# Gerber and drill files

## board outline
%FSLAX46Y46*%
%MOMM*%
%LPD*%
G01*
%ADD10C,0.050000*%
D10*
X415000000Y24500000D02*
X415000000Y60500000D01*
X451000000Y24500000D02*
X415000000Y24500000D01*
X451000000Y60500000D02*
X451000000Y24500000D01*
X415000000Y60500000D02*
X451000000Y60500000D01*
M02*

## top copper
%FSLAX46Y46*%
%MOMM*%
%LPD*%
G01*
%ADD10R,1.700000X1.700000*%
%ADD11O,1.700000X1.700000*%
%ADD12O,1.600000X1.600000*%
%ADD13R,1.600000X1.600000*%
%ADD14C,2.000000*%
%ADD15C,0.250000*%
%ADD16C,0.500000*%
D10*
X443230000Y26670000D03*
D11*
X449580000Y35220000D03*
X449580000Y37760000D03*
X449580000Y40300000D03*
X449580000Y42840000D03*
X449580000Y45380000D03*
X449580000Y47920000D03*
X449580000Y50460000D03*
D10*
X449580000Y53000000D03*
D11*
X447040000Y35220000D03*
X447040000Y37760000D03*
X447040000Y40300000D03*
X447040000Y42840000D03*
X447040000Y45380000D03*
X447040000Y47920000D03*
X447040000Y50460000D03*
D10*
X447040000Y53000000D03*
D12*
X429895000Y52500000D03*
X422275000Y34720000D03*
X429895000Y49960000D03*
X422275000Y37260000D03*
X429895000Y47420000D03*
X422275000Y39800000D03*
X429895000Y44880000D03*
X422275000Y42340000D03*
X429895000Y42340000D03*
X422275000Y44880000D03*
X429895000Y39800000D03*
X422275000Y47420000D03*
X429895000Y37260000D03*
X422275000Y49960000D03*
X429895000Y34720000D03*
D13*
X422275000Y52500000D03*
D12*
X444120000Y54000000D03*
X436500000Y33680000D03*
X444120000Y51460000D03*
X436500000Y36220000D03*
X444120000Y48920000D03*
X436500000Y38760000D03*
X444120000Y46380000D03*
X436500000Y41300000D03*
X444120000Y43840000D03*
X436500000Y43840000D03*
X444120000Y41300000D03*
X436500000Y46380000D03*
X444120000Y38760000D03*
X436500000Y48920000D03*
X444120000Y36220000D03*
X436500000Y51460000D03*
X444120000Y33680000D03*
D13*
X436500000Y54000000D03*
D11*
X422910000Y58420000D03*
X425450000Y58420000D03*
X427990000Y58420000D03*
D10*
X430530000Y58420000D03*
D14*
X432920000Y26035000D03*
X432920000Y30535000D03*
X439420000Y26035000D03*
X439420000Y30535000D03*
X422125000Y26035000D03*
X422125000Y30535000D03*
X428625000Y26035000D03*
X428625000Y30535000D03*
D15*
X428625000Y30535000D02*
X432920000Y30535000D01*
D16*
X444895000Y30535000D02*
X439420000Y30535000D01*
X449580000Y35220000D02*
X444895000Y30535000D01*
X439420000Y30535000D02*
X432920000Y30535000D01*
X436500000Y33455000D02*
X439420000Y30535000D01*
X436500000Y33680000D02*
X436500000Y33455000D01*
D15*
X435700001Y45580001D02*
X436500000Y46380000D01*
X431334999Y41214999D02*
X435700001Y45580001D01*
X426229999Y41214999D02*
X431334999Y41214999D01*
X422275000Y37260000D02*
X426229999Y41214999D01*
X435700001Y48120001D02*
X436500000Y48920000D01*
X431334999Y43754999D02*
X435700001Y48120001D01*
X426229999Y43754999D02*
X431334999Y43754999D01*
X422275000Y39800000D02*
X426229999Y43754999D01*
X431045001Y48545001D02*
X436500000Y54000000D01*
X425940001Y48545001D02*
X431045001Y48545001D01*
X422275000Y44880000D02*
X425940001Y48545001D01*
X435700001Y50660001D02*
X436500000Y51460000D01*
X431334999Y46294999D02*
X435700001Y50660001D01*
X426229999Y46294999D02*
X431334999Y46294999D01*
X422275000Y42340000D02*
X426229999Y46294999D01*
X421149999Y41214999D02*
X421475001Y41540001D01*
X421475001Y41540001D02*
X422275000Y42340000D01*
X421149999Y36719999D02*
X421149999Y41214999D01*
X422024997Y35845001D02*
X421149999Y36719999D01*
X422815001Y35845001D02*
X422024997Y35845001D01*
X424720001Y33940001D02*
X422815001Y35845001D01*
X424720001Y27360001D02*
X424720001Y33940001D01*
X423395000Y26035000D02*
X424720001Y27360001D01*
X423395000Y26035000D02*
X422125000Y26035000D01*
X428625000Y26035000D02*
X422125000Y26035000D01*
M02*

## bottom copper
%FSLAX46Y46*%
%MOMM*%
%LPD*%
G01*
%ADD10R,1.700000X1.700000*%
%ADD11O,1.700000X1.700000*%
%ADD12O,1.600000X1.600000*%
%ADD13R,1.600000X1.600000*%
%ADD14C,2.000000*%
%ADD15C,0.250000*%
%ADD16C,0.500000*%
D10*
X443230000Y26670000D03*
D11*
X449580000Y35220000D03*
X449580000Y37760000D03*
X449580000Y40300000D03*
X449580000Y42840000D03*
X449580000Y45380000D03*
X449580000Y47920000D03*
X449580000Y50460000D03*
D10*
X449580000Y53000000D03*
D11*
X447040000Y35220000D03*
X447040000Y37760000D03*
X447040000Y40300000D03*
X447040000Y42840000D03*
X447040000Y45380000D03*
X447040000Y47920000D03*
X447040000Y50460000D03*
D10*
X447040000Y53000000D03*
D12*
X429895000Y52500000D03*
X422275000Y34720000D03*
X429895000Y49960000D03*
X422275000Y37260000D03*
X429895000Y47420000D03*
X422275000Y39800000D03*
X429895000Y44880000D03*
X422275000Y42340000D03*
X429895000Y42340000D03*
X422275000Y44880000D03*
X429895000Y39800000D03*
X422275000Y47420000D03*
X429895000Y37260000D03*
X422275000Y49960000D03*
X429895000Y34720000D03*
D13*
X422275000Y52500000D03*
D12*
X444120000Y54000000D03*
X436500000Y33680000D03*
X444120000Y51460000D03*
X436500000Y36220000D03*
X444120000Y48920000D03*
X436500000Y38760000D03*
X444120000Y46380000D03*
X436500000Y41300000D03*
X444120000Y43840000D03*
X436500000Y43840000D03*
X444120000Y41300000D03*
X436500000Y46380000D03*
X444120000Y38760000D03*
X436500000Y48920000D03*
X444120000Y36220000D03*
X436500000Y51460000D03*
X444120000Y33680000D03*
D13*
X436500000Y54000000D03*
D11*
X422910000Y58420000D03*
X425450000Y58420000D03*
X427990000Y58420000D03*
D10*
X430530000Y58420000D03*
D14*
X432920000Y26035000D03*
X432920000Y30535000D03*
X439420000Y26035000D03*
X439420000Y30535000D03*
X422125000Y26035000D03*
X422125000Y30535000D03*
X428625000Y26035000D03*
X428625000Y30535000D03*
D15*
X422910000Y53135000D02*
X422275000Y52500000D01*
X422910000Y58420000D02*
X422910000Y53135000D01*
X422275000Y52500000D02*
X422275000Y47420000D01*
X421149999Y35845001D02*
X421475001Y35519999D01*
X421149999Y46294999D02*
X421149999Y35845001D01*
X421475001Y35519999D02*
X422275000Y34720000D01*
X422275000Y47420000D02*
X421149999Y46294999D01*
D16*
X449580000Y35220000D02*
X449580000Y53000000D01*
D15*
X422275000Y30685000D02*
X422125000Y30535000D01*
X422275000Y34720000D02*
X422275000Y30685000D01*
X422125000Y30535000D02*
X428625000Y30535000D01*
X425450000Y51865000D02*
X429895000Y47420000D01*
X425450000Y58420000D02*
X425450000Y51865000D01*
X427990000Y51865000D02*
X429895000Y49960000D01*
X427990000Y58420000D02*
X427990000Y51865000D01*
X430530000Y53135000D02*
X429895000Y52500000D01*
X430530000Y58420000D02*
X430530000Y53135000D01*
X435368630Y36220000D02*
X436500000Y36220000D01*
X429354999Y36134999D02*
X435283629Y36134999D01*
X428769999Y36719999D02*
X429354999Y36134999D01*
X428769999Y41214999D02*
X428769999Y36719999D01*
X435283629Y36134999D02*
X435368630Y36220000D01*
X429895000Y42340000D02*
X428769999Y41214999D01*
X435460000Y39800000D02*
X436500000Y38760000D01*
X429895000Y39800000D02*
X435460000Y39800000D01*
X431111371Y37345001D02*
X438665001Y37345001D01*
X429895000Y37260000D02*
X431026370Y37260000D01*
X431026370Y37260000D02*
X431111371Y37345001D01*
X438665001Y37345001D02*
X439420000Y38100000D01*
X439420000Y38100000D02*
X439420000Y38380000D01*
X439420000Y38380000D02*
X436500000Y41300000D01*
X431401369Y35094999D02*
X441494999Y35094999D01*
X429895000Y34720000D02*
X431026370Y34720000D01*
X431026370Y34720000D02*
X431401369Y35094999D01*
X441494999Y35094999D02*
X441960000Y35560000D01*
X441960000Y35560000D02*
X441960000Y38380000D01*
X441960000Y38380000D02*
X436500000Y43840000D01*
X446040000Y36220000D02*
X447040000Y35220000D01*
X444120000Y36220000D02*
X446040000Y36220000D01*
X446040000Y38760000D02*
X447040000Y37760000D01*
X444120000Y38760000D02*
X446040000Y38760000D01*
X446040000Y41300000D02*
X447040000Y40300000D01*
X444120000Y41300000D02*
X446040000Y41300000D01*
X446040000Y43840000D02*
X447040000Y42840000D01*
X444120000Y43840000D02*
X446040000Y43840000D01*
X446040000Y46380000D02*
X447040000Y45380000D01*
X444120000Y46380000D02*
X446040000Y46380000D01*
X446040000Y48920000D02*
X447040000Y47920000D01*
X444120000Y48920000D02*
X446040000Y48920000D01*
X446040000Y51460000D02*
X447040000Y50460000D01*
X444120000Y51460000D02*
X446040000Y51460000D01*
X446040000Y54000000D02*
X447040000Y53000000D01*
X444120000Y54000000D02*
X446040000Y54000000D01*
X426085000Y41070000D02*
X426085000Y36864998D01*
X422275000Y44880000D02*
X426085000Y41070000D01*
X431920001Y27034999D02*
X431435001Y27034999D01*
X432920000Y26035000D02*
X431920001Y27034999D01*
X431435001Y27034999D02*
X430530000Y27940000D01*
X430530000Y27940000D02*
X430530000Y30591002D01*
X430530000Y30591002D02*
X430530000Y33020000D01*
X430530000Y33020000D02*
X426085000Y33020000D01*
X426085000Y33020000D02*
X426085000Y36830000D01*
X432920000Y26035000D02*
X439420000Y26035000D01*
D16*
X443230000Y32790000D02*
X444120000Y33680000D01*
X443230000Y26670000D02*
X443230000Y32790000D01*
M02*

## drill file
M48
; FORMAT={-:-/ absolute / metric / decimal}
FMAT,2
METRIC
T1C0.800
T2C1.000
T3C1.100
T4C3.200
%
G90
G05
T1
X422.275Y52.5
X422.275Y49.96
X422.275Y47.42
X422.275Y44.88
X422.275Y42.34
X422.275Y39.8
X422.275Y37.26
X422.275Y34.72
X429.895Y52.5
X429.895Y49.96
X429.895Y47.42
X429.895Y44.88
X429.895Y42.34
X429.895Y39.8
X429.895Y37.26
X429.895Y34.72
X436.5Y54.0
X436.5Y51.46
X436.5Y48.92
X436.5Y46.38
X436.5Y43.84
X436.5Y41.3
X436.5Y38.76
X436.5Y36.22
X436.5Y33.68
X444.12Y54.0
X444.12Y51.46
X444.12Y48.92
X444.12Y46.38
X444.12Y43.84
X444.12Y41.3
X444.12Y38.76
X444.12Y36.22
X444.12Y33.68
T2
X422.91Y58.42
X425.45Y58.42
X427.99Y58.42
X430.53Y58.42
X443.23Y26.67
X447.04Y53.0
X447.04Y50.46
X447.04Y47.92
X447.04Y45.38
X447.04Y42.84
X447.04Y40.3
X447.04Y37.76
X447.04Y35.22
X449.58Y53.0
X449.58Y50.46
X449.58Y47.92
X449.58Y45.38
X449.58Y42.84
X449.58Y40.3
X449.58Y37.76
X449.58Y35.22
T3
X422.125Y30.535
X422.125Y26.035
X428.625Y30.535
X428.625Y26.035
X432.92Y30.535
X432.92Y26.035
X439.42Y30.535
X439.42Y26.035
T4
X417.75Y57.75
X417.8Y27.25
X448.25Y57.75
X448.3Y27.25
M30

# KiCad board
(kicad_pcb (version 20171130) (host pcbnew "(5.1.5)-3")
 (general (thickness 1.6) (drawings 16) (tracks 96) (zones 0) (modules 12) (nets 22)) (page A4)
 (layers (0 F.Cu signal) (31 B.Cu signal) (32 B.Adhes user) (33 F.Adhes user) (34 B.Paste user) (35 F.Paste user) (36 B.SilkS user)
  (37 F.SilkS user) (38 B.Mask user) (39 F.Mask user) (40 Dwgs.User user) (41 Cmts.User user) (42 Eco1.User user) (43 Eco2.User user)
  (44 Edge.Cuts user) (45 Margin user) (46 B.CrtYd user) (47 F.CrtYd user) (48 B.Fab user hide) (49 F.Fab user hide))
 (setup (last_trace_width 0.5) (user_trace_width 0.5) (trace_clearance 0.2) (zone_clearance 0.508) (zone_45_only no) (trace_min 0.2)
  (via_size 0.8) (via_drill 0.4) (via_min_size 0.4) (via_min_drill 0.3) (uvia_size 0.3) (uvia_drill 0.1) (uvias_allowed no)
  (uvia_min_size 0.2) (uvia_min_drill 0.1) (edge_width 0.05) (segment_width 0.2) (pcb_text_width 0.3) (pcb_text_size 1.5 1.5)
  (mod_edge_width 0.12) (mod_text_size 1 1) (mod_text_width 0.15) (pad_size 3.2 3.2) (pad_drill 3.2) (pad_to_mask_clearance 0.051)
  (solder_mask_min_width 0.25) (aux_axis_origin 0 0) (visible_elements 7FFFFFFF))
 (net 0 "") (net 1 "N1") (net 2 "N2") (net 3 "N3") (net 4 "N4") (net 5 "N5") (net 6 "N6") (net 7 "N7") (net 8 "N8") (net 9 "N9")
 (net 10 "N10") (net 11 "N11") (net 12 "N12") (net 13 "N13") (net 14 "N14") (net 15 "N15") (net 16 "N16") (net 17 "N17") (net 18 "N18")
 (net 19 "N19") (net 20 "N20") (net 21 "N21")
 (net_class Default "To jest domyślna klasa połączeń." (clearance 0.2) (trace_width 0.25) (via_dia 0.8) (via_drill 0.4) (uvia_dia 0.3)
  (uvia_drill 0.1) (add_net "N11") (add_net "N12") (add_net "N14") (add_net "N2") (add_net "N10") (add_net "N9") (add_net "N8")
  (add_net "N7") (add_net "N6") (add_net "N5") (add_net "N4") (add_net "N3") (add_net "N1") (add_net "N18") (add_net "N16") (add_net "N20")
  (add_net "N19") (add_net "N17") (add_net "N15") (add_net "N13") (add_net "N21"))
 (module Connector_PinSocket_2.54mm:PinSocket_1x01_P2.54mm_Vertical (layer F.Cu) (at 443.23 -26.67)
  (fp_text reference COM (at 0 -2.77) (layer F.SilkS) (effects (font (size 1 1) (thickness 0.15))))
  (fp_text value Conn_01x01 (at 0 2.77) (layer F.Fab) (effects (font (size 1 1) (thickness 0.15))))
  (pad 1 thru_hole rect (at 0 0) (size 1.7 1.7) (drill 1) (layers *.Cu *.Mask) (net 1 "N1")))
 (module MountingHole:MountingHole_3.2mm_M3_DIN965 (layer F.Cu) (at 448.3 -27.25)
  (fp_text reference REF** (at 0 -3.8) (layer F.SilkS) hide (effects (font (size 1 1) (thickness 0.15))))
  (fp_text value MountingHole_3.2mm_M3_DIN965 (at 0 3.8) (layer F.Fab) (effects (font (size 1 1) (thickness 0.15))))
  (pad "" np_thru_hole circle (at 0 0) (size 3.2 3.2) (drill 3.2) (layers *.Cu)))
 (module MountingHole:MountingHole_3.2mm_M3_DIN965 (layer F.Cu) (at 417.8 -27.25)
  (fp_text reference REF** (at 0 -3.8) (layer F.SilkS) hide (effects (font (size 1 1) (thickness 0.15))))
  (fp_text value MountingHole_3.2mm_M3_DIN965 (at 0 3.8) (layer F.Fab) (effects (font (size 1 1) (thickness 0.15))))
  (pad "" np_thru_hole circle (at 0 0) (size 3.2 3.2) (drill 3.2) (layers *.Cu)))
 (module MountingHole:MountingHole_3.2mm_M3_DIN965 (layer F.Cu) (at 448.25 -57.75)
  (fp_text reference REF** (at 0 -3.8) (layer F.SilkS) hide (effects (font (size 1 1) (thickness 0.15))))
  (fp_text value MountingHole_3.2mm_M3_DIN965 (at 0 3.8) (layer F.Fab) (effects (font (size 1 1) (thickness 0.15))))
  (pad "" np_thru_hole circle (at 0 0) (size 3.2 3.2) (drill 3.2) (layers *.Cu)))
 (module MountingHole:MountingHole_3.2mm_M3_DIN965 (layer F.Cu) (at 417.75 -57.75)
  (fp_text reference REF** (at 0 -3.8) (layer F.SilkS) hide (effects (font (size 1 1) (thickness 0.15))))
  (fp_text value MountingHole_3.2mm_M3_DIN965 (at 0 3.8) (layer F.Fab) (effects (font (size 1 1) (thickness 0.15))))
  (pad "" np_thru_hole circle (at 0 0) (size 3.2 3.2) (drill 3.2) (layers *.Cu)))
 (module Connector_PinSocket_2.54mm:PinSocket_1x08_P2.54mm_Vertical (layer F.Cu) (at 449.58 -53)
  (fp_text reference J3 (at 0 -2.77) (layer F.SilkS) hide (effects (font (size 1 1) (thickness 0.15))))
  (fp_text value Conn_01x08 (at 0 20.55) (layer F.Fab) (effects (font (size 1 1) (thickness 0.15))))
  (pad 8 thru_hole oval (at 0 17.78) (size 1.7 1.7) (drill 1) (layers *.Cu *.Mask) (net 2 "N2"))
  (pad 7 thru_hole oval (at 0 15.24) (size 1.7 1.7) (drill 1) (layers *.Cu *.Mask) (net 2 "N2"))
  (pad 6 thru_hole oval (at 0 12.7) (size 1.7 1.7) (drill 1) (layers *.Cu *.Mask) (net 2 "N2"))
  (pad 5 thru_hole oval (at 0 10.16) (size 1.7 1.7) (drill 1) (layers *.Cu *.Mask) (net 2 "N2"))
  (pad 4 thru_hole oval (at 0 7.62) (size 1.7 1.7) (drill 1) (layers *.Cu *.Mask) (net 2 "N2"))
  (pad 3 thru_hole oval (at 0 5.08) (size 1.7 1.7) (drill 1) (layers *.Cu *.Mask) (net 2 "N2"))
  (pad 2 thru_hole oval (at 0 2.54) (size 1.7 1.7) (drill 1) (layers *.Cu *.Mask) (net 2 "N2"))
  (pad 1 thru_hole rect (at 0 0) (size 1.7 1.7) (drill 1) (layers *.Cu *.Mask) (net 2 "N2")))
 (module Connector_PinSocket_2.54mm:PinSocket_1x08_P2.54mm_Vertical (layer F.Cu) (at 447.04 -53)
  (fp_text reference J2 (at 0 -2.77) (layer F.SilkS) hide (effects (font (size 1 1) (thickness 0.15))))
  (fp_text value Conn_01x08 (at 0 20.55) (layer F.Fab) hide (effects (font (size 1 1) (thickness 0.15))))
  (pad 8 thru_hole oval (at 0 17.78) (size 1.7 1.7) (drill 1) (layers *.Cu *.Mask) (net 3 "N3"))
  (pad 7 thru_hole oval (at 0 15.24) (size 1.7 1.7) (drill 1) (layers *.Cu *.Mask) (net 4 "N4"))
  (pad 6 thru_hole oval (at 0 12.7) (size 1.7 1.7) (drill 1) (layers *.Cu *.Mask) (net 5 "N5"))
  (pad 5 thru_hole oval (at 0 10.16) (size 1.7 1.7) (drill 1) (layers *.Cu *.Mask) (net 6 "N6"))
  (pad 4 thru_hole oval (at 0 7.62) (size 1.7 1.7) (drill 1) (layers *.Cu *.Mask) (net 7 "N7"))
  (pad 3 thru_hole oval (at 0 5.08) (size 1.7 1.7) (drill 1) (layers *.Cu *.Mask) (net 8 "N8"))
  (pad 2 thru_hole oval (at 0 2.54) (size 1.7 1.7) (drill 1) (layers *.Cu *.Mask) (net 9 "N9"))
  (pad 1 thru_hole rect (at 0 0) (size 1.7 1.7) (drill 1) (layers *.Cu *.Mask) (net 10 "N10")))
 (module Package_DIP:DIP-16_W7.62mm (layer F.Cu) (at 422.275 -52.5)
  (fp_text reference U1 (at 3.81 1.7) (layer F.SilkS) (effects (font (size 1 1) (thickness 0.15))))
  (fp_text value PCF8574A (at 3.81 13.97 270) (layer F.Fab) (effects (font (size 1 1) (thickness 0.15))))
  (pad 16 thru_hole oval (at 7.62 0) (size 1.6 1.6) (drill 0.8) (layers *.Cu *.Mask) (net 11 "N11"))
  (pad 8 thru_hole oval (at 0 17.78) (size 1.6 1.6) (drill 0.8) (layers *.Cu *.Mask) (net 2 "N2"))
  (pad 15 thru_hole oval (at 7.62 2.54) (size 1.6 1.6) (drill 0.8) (layers *.Cu *.Mask) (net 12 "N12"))
  (pad 7 thru_hole oval (at 0 15.24) (size 1.6 1.6) (drill 0.8) (layers *.Cu *.Mask) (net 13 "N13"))
  (pad 14 thru_hole oval (at 7.62 5.08) (size 1.6 1.6) (drill 0.8) (layers *.Cu *.Mask) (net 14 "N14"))
  (pad 6 thru_hole oval (at 0 12.7) (size 1.6 1.6) (drill 0.8) (layers *.Cu *.Mask) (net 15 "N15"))
  (pad 13 thru_hole oval (at 7.62 7.62) (size 1.6 1.6) (drill 0.8) (layers *.Cu *.Mask))
  (pad 5 thru_hole oval (at 0 10.16) (size 1.6 1.6) (drill 0.8) (layers *.Cu *.Mask) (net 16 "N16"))
  (pad 12 thru_hole oval (at 7.62 10.16) (size 1.6 1.6) (drill 0.8) (layers *.Cu *.Mask) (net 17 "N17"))
  (pad 4 thru_hole oval (at 0 7.62) (size 1.6 1.6) (drill 0.8) (layers *.Cu *.Mask) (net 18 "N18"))
  (pad 11 thru_hole oval (at 7.62 12.7) (size 1.6 1.6) (drill 0.8) (layers *.Cu *.Mask) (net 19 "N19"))
  (pad 3 thru_hole oval (at 0 5.08) (size 1.6 1.6) (drill 0.8) (layers *.Cu *.Mask) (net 2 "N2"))
  (pad 10 thru_hole oval (at 7.62 15.24) (size 1.6 1.6) (drill 0.8) (layers *.Cu *.Mask) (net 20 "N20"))
  (pad 2 thru_hole oval (at 0 2.54) (size 1.6 1.6) (drill 0.8) (layers *.Cu *.Mask) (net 2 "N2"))
  (pad 9 thru_hole oval (at 7.62 17.78) (size 1.6 1.6) (drill 0.8) (layers *.Cu *.Mask) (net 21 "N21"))
  (pad 1 thru_hole rect (at 0 0) (size 1.6 1.6) (drill 0.8) (layers *.Cu *.Mask) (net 2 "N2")))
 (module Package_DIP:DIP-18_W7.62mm (layer F.Cu) (at 436.5 -54)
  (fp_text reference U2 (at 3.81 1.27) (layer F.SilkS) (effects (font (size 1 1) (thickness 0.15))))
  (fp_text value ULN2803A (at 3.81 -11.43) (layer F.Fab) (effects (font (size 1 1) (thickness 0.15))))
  (pad 18 thru_hole oval (at 7.62 0) (size 1.6 1.6) (drill 0.8) (layers *.Cu *.Mask) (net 10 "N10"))
  (pad 9 thru_hole oval (at 0 20.32) (size 1.6 1.6) (drill 0.8) (layers *.Cu *.Mask) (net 2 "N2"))
  (pad 17 thru_hole oval (at 7.62 2.54) (size 1.6 1.6) (drill 0.8) (layers *.Cu *.Mask) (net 9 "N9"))
  (pad 8 thru_hole oval (at 0 17.78) (size 1.6 1.6) (drill 0.8) (layers *.Cu *.Mask) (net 17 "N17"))
  (pad 16 thru_hole oval (at 7.62 5.08) (size 1.6 1.6) (drill 0.8) (layers *.Cu *.Mask) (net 8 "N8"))
  (pad 7 thru_hole oval (at 0 15.24) (size 1.6 1.6) (drill 0.8) (layers *.Cu *.Mask) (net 19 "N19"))
  (pad 15 thru_hole oval (at 7.62 7.62) (size 1.6 1.6) (drill 0.8) (layers *.Cu *.Mask) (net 7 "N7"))
  (pad 6 thru_hole oval (at 0 12.7) (size 1.6 1.6) (drill 0.8) (layers *.Cu *.Mask) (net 20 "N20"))
  (pad 14 thru_hole oval (at 7.62 10.16) (size 1.6 1.6) (drill 0.8) (layers *.Cu *.Mask) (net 6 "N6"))
  (pad 5 thru_hole oval (at 0 10.16) (size 1.6 1.6) (drill 0.8) (layers *.Cu *.Mask) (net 21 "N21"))
  (pad 13 thru_hole oval (at 7.62 12.7) (size 1.6 1.6) (drill 0.8) (layers *.Cu *.Mask) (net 5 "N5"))
  (pad 4 thru_hole oval (at 0 7.62) (size 1.6 1.6) (drill 0.8) (layers *.Cu *.Mask) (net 13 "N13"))
  (pad 12 thru_hole oval (at 7.62 15.24) (size 1.6 1.6) (drill 0.8) (layers *.Cu *.Mask) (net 4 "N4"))
  (pad 3 thru_hole oval (at 0 5.08) (size 1.6 1.6) (drill 0.8) (layers *.Cu *.Mask) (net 15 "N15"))
  (pad 11 thru_hole oval (at 7.62 17.78) (size 1.6 1.6) (drill 0.8) (layers *.Cu *.Mask) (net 3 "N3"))
  (pad 2 thru_hole oval (at 0 2.54) (size 1.6 1.6) (drill 0.8) (layers *.Cu *.Mask) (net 16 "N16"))
  (pad 10 thru_hole oval (at 7.62 20.32) (size 1.6 1.6) (drill 0.8) (layers *.Cu *.Mask) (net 1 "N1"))
  (pad 1 thru_hole rect (at 0 0) (size 1.6 1.6) (drill 0.8) (layers *.Cu *.Mask) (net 18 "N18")))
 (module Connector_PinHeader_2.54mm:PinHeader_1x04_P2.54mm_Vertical (layer F.Cu) (at 430.53 -58.42 270)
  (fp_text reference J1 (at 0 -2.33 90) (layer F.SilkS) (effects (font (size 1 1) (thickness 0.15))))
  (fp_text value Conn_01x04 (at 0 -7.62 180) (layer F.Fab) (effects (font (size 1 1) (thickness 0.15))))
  (pad 4 thru_hole oval (at 0 7.62 270) (size 1.7 1.7) (drill 1) (layers *.Cu *.Mask) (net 2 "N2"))
  (pad 3 thru_hole oval (at 0 5.08 270) (size 1.7 1.7) (drill 1) (layers *.Cu *.Mask) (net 14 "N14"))
  (pad 2 thru_hole oval (at 0 2.54 270) (size 1.7 1.7) (drill 1) (layers *.Cu *.Mask) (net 12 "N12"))
  (pad 1 thru_hole rect (at 0 0 270) (size 1.7 1.7) (drill 1) (layers *.Cu *.Mask) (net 11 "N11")))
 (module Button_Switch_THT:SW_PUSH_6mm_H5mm (layer F.Cu) (at 439.42 -26.035 180)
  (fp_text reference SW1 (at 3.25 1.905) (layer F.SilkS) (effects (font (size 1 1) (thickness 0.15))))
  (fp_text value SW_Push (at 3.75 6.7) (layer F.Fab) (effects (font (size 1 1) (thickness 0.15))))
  (pad 1 thru_hole circle (at 6.5 0 270) (size 2 2) (drill 1.1) (layers *.Cu *.Mask) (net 18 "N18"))
  (pad 2 thru_hole circle (at 6.5 4.5 270) (size 2 2) (drill 1.1) (layers *.Cu *.Mask) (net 2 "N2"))
  (pad 1 thru_hole circle (at 0 0 270) (size 2 2) (drill 1.1) (layers *.Cu *.Mask) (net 18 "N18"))
  (pad 2 thru_hole circle (at 0 4.5 270) (size 2 2) (drill 1.1) (layers *.Cu *.Mask) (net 2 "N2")))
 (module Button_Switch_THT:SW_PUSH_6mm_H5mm (layer F.Cu) (at 428.625 -26.035 180)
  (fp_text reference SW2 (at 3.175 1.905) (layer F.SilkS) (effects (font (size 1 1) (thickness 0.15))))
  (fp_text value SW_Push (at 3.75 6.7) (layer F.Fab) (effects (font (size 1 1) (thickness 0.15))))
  (pad 1 thru_hole circle (at 6.5 0 270) (size 2 2) (drill 1.1) (layers *.Cu *.Mask) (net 16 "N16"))
  (pad 2 thru_hole circle (at 6.5 4.5 270) (size 2 2) (drill 1.1) (layers *.Cu *.Mask) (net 2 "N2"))
  (pad 1 thru_hole circle (at 0 0 270) (size 2 2) (drill 1.1) (layers *.Cu *.Mask) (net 16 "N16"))
  (pad 2 thru_hole circle (at 0 4.5 270) (size 2 2) (drill 1.1) (layers *.Cu *.Mask) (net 2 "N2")))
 (gr_line (start 415 -24.5) (end 415 -60.5) (layer Edge.Cuts) (width 0.05))
 (gr_line (start 451 -24.5) (end 415 -24.5) (layer Edge.Cuts) (width 0.05))
 (gr_line (start 451 -60.5) (end 451 -24.5) (layer Edge.Cuts) (width 0.05))
 (gr_line (start 415 -60.5) (end 451 -60.5) (layer Edge.Cuts) (width 0.05))
 (segment (start 422.91 -53.135) (end 422.275 -52.5) (width 0.25) (layer B.Cu) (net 2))
 (segment (start 422.91 -58.42) (end 422.91 -53.135) (width 0.25) (layer B.Cu) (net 2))
 (segment (start 422.275 -52.5) (end 422.275 -47.42) (width 0.25) (layer B.Cu) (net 2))
 (segment (start 421.149999 -35.845001) (end 421.475001 -35.519999) (width 0.25) (layer B.Cu) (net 2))
 (segment (start 421.149999 -46.294999) (end 421.149999 -35.845001) (width 0.25) (layer B.Cu) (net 2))
 (segment (start 421.475001 -35.519999) (end 422.275 -34.72) (width 0.25) (layer B.Cu) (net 2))
 (segment (start 422.275 -47.42) (end 421.149999 -46.294999) (width 0.25) (layer B.Cu) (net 2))
 (segment (start 449.58 -35.22) (end 449.58 -53) (width 0.5) (layer B.Cu) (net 2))
 (segment (start 422.275 -30.685) (end 422.125 -30.535) (width 0.25) (layer B.Cu) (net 2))
 (segment (start 422.275 -34.72) (end 422.275 -30.685) (width 0.25) (layer B.Cu) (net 2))
 (segment (start 422.125 -30.535) (end 428.625 -30.535) (width 0.25) (layer B.Cu) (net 2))
 (segment (start 428.625 -30.535) (end 432.92 -30.535) (width 0.25) (layer F.Cu) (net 2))
 (segment (start 444.895 -30.535) (end 439.42 -30.535) (width 0.5) (layer F.Cu) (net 2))
 (segment (start 449.58 -35.22) (end 444.895 -30.535) (width 0.5) (layer F.Cu) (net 2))
 (segment (start 439.42 -30.535) (end 432.92 -30.535) (width 0.5) (layer F.Cu) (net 2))
 (segment (start 436.5 -33.455) (end 439.42 -30.535) (width 0.5) (layer F.Cu) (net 2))
 (segment (start 436.5 -33.68) (end 436.5 -33.455) (width 0.5) (layer F.Cu) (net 2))
 (segment (start 425.45 -51.865) (end 429.895 -47.42) (width 0.25) (layer B.Cu) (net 14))
 (segment (start 425.45 -58.42) (end 425.45 -51.865) (width 0.25) (layer B.Cu) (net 14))
 (segment (start 427.99 -51.865) (end 429.895 -49.96) (width 0.25) (layer B.Cu) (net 12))
 (segment (start 427.99 -58.42) (end 427.99 -51.865) (width 0.25) (layer B.Cu) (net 12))
 (segment (start 430.53 -53.135) (end 429.895 -52.5) (width 0.25) (layer B.Cu) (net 11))
 (segment (start 430.53 -58.42) (end 430.53 -53.135) (width 0.25) (layer B.Cu) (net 11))
 (segment (start 435.700001 -45.580001) (end 436.5 -46.38) (width 0.25) (layer F.Cu) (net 13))
 (segment (start 431.334999 -41.214999) (end 435.700001 -45.580001) (width 0.25) (layer F.Cu) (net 13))
 (segment (start 426.229999 -41.214999) (end 431.334999 -41.214999) (width 0.25) (layer F.Cu) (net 13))
 (segment (start 422.275 -37.26) (end 426.229999 -41.214999) (width 0.25) (layer F.Cu) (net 13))
 (segment (start 435.700001 -48.120001) (end 436.5 -48.92) (width 0.25) (layer F.Cu) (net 15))
 (segment (start 431.334999 -43.754999) (end 435.700001 -48.120001) (width 0.25) (layer F.Cu) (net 15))
 (segment (start 426.229999 -43.754999) (end 431.334999 -43.754999) (width 0.25) (layer F.Cu) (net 15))
 (segment (start 422.275 -39.8) (end 426.229999 -43.754999) (width 0.25) (layer F.Cu) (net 15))
 (segment (start 435.36863 -36.22) (end 436.5 -36.22) (width 0.25) (layer B.Cu) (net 17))
 (segment (start 429.354999 -36.134999) (end 435.283629 -36.134999) (width 0.25) (layer B.Cu) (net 17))
 (segment (start 428.769999 -36.719999) (end 429.354999 -36.134999) (width 0.25) (layer B.Cu) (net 17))
 (segment (start 428.769999 -41.214999) (end 428.769999 -36.719999) (width 0.25) (layer B.Cu) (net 17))
 (segment (start 435.283629 -36.134999) (end 435.36863 -36.22) (width 0.25) (layer B.Cu) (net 17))
 (segment (start 429.895 -42.34) (end 428.769999 -41.214999) (width 0.25) (layer B.Cu) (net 17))
 (segment (start 435.46 -39.8) (end 436.5 -38.76) (width 0.25) (layer B.Cu) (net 19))
 (segment (start 429.895 -39.8) (end 435.46 -39.8) (width 0.25) (layer B.Cu) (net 19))
 (segment (start 431.111371 -37.345001) (end 438.665001 -37.345001) (width 0.25) (layer B.Cu) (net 20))
 (segment (start 429.895 -37.26) (end 431.02637 -37.26) (width 0.25) (layer B.Cu) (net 20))
 (segment (start 431.02637 -37.26) (end 431.111371 -37.345001) (width 0.25) (layer B.Cu) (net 20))
 (segment (start 438.665001 -37.345001) (end 439.42 -38.1) (width 0.25) (layer B.Cu) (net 20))
 (segment (start 439.42 -38.1) (end 439.42 -38.38) (width 0.25) (layer B.Cu) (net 20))
 (segment (start 439.42 -38.38) (end 436.5 -41.3) (width 0.25) (layer B.Cu) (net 20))
 (segment (start 431.401369 -35.094999) (end 441.494999 -35.094999) (width 0.25) (layer B.Cu) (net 21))
 (segment (start 429.895 -34.72) (end 431.02637 -34.72) (width 0.25) (layer B.Cu) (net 21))
 (segment (start 431.02637 -34.72) (end 431.401369 -35.094999) (width 0.25) (layer B.Cu) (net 21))
 (segment (start 441.494999 -35.094999) (end 441.96 -35.56) (width 0.25) (layer B.Cu) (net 21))
 (segment (start 441.96 -35.56) (end 441.96 -38.38) (width 0.25) (layer B.Cu) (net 21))
 (segment (start 441.96 -38.38) (end 436.5 -43.84) (width 0.25) (layer B.Cu) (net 21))
 (segment (start 446.04 -36.22) (end 447.04 -35.22) (width 0.25) (layer B.Cu) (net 3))
 (segment (start 444.12 -36.22) (end 446.04 -36.22) (width 0.25) (layer B.Cu) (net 3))
 (segment (start 446.04 -38.76) (end 447.04 -37.76) (width 0.25) (layer B.Cu) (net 4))
 (segment (start 444.12 -38.76) (end 446.04 -38.76) (width 0.25) (layer B.Cu) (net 4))
 (segment (start 446.04 -41.3) (end 447.04 -40.3) (width 0.25) (layer B.Cu) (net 5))
 (segment (start 444.12 -41.3) (end 446.04 -41.3) (width 0.25) (layer B.Cu) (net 5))
 (segment (start 446.04 -43.84) (end 447.04 -42.84) (width 0.25) (layer B.Cu) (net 6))
 (segment (start 444.12 -43.84) (end 446.04 -43.84) (width 0.25) (layer B.Cu) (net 6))
 (segment (start 446.04 -46.38) (end 447.04 -45.38) (width 0.25) (layer B.Cu) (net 7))
 (segment (start 444.12 -46.38) (end 446.04 -46.38) (width 0.25) (layer B.Cu) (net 7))
 (segment (start 446.04 -48.92) (end 447.04 -47.92) (width 0.25) (layer B.Cu) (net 8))
 (segment (start 444.12 -48.92) (end 446.04 -48.92) (width 0.25) (layer B.Cu) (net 8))
 (segment (start 446.04 -51.46) (end 447.04 -50.46) (width 0.25) (layer B.Cu) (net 9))
 (segment (start 444.12 -51.46) (end 446.04 -51.46) (width 0.25) (layer B.Cu) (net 9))
 (segment (start 446.04 -54) (end 447.04 -53) (width 0.25) (layer B.Cu) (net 10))
 (segment (start 444.12 -54) (end 446.04 -54) (width 0.25) (layer B.Cu) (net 10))
 (segment (start 431.045001 -48.545001) (end 436.5 -54) (width 0.25) (layer F.Cu) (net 18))
 (segment (start 425.940001 -48.545001) (end 431.045001 -48.545001) (width 0.25) (layer F.Cu) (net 18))
 (segment (start 422.275 -44.88) (end 425.940001 -48.545001) (width 0.25) (layer F.Cu) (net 18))
 (segment (start 426.085 -41.07) (end 426.085 -36.864998) (width 0.25) (layer B.Cu) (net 18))
 (segment (start 422.275 -44.88) (end 426.085 -41.07) (width 0.25) (layer B.Cu) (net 18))
 (segment (start 431.920001 -27.034999) (end 431.435001 -27.034999) (width 0.25) (layer B.Cu) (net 18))
 (segment (start 432.92 -26.035) (end 431.920001 -27.034999) (width 0.25) (layer B.Cu) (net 18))
 (segment (start 431.435001 -27.034999) (end 430.53 -27.94) (width 0.25) (layer B.Cu) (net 18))
 (segment (start 430.53 -27.94) (end 430.53 -30.591002) (width 0.25) (layer B.Cu) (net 18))
 (segment (start 430.53 -30.591002) (end 430.53 -33.02) (width 0.25) (layer B.Cu) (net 18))
 (segment (start 430.53 -33.02) (end 426.085 -33.02) (width 0.25) (layer B.Cu) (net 18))
 (segment (start 426.085 -33.02) (end 426.085 -36.83) (width 0.25) (layer B.Cu) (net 18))
 (segment (start 432.92 -26.035) (end 439.42 -26.035) (width 0.25) (layer B.Cu) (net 18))
 (segment (start 435.700001 -50.660001) (end 436.5 -51.46) (width 0.25) (layer F.Cu) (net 16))
 (segment (start 431.334999 -46.294999) (end 435.700001 -50.660001) (width 0.25) (layer F.Cu) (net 16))
 (segment (start 426.229999 -46.294999) (end 431.334999 -46.294999) (width 0.25) (layer F.Cu) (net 16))
 (segment (start 422.275 -42.34) (end 426.229999 -46.294999) (width 0.25) (layer F.Cu) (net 16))
 (segment (start 421.149999 -41.214999) (end 421.475001 -41.540001) (width 0.25) (layer F.Cu) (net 16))
 (segment (start 421.475001 -41.540001) (end 422.275 -42.34) (width 0.25) (layer F.Cu) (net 16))
 (segment (start 421.149999 -36.719999) (end 421.149999 -41.214999) (width 0.25) (layer F.Cu) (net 16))
 (segment (start 422.024997 -35.845001) (end 421.149999 -36.719999) (width 0.25) (layer F.Cu) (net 16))
 (segment (start 422.815001 -35.845001) (end 422.024997 -35.845001) (width 0.25) (layer F.Cu) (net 16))
 (segment (start 424.720001 -33.940001) (end 422.815001 -35.845001) (width 0.25) (layer F.Cu) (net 16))
 (segment (start 424.720001 -27.360001) (end 424.720001 -33.940001) (width 0.25) (layer F.Cu) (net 16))
 (segment (start 423.395 -26.035) (end 424.720001 -27.360001) (width 0.25) (layer F.Cu) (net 16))
 (segment (start 423.395 -26.035) (end 422.125 -26.035) (width 0.25) (layer F.Cu) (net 16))
 (segment (start 428.625 -26.035) (end 422.125 -26.035) (width 0.25) (layer F.Cu) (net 16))
 (segment (start 443.23 -32.79) (end 444.12 -33.68) (width 0.5) (layer B.Cu) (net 1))
 (segment (start 443.23 -26.67) (end 443.23 -32.79) (width 0.5) (layer B.Cu) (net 1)))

